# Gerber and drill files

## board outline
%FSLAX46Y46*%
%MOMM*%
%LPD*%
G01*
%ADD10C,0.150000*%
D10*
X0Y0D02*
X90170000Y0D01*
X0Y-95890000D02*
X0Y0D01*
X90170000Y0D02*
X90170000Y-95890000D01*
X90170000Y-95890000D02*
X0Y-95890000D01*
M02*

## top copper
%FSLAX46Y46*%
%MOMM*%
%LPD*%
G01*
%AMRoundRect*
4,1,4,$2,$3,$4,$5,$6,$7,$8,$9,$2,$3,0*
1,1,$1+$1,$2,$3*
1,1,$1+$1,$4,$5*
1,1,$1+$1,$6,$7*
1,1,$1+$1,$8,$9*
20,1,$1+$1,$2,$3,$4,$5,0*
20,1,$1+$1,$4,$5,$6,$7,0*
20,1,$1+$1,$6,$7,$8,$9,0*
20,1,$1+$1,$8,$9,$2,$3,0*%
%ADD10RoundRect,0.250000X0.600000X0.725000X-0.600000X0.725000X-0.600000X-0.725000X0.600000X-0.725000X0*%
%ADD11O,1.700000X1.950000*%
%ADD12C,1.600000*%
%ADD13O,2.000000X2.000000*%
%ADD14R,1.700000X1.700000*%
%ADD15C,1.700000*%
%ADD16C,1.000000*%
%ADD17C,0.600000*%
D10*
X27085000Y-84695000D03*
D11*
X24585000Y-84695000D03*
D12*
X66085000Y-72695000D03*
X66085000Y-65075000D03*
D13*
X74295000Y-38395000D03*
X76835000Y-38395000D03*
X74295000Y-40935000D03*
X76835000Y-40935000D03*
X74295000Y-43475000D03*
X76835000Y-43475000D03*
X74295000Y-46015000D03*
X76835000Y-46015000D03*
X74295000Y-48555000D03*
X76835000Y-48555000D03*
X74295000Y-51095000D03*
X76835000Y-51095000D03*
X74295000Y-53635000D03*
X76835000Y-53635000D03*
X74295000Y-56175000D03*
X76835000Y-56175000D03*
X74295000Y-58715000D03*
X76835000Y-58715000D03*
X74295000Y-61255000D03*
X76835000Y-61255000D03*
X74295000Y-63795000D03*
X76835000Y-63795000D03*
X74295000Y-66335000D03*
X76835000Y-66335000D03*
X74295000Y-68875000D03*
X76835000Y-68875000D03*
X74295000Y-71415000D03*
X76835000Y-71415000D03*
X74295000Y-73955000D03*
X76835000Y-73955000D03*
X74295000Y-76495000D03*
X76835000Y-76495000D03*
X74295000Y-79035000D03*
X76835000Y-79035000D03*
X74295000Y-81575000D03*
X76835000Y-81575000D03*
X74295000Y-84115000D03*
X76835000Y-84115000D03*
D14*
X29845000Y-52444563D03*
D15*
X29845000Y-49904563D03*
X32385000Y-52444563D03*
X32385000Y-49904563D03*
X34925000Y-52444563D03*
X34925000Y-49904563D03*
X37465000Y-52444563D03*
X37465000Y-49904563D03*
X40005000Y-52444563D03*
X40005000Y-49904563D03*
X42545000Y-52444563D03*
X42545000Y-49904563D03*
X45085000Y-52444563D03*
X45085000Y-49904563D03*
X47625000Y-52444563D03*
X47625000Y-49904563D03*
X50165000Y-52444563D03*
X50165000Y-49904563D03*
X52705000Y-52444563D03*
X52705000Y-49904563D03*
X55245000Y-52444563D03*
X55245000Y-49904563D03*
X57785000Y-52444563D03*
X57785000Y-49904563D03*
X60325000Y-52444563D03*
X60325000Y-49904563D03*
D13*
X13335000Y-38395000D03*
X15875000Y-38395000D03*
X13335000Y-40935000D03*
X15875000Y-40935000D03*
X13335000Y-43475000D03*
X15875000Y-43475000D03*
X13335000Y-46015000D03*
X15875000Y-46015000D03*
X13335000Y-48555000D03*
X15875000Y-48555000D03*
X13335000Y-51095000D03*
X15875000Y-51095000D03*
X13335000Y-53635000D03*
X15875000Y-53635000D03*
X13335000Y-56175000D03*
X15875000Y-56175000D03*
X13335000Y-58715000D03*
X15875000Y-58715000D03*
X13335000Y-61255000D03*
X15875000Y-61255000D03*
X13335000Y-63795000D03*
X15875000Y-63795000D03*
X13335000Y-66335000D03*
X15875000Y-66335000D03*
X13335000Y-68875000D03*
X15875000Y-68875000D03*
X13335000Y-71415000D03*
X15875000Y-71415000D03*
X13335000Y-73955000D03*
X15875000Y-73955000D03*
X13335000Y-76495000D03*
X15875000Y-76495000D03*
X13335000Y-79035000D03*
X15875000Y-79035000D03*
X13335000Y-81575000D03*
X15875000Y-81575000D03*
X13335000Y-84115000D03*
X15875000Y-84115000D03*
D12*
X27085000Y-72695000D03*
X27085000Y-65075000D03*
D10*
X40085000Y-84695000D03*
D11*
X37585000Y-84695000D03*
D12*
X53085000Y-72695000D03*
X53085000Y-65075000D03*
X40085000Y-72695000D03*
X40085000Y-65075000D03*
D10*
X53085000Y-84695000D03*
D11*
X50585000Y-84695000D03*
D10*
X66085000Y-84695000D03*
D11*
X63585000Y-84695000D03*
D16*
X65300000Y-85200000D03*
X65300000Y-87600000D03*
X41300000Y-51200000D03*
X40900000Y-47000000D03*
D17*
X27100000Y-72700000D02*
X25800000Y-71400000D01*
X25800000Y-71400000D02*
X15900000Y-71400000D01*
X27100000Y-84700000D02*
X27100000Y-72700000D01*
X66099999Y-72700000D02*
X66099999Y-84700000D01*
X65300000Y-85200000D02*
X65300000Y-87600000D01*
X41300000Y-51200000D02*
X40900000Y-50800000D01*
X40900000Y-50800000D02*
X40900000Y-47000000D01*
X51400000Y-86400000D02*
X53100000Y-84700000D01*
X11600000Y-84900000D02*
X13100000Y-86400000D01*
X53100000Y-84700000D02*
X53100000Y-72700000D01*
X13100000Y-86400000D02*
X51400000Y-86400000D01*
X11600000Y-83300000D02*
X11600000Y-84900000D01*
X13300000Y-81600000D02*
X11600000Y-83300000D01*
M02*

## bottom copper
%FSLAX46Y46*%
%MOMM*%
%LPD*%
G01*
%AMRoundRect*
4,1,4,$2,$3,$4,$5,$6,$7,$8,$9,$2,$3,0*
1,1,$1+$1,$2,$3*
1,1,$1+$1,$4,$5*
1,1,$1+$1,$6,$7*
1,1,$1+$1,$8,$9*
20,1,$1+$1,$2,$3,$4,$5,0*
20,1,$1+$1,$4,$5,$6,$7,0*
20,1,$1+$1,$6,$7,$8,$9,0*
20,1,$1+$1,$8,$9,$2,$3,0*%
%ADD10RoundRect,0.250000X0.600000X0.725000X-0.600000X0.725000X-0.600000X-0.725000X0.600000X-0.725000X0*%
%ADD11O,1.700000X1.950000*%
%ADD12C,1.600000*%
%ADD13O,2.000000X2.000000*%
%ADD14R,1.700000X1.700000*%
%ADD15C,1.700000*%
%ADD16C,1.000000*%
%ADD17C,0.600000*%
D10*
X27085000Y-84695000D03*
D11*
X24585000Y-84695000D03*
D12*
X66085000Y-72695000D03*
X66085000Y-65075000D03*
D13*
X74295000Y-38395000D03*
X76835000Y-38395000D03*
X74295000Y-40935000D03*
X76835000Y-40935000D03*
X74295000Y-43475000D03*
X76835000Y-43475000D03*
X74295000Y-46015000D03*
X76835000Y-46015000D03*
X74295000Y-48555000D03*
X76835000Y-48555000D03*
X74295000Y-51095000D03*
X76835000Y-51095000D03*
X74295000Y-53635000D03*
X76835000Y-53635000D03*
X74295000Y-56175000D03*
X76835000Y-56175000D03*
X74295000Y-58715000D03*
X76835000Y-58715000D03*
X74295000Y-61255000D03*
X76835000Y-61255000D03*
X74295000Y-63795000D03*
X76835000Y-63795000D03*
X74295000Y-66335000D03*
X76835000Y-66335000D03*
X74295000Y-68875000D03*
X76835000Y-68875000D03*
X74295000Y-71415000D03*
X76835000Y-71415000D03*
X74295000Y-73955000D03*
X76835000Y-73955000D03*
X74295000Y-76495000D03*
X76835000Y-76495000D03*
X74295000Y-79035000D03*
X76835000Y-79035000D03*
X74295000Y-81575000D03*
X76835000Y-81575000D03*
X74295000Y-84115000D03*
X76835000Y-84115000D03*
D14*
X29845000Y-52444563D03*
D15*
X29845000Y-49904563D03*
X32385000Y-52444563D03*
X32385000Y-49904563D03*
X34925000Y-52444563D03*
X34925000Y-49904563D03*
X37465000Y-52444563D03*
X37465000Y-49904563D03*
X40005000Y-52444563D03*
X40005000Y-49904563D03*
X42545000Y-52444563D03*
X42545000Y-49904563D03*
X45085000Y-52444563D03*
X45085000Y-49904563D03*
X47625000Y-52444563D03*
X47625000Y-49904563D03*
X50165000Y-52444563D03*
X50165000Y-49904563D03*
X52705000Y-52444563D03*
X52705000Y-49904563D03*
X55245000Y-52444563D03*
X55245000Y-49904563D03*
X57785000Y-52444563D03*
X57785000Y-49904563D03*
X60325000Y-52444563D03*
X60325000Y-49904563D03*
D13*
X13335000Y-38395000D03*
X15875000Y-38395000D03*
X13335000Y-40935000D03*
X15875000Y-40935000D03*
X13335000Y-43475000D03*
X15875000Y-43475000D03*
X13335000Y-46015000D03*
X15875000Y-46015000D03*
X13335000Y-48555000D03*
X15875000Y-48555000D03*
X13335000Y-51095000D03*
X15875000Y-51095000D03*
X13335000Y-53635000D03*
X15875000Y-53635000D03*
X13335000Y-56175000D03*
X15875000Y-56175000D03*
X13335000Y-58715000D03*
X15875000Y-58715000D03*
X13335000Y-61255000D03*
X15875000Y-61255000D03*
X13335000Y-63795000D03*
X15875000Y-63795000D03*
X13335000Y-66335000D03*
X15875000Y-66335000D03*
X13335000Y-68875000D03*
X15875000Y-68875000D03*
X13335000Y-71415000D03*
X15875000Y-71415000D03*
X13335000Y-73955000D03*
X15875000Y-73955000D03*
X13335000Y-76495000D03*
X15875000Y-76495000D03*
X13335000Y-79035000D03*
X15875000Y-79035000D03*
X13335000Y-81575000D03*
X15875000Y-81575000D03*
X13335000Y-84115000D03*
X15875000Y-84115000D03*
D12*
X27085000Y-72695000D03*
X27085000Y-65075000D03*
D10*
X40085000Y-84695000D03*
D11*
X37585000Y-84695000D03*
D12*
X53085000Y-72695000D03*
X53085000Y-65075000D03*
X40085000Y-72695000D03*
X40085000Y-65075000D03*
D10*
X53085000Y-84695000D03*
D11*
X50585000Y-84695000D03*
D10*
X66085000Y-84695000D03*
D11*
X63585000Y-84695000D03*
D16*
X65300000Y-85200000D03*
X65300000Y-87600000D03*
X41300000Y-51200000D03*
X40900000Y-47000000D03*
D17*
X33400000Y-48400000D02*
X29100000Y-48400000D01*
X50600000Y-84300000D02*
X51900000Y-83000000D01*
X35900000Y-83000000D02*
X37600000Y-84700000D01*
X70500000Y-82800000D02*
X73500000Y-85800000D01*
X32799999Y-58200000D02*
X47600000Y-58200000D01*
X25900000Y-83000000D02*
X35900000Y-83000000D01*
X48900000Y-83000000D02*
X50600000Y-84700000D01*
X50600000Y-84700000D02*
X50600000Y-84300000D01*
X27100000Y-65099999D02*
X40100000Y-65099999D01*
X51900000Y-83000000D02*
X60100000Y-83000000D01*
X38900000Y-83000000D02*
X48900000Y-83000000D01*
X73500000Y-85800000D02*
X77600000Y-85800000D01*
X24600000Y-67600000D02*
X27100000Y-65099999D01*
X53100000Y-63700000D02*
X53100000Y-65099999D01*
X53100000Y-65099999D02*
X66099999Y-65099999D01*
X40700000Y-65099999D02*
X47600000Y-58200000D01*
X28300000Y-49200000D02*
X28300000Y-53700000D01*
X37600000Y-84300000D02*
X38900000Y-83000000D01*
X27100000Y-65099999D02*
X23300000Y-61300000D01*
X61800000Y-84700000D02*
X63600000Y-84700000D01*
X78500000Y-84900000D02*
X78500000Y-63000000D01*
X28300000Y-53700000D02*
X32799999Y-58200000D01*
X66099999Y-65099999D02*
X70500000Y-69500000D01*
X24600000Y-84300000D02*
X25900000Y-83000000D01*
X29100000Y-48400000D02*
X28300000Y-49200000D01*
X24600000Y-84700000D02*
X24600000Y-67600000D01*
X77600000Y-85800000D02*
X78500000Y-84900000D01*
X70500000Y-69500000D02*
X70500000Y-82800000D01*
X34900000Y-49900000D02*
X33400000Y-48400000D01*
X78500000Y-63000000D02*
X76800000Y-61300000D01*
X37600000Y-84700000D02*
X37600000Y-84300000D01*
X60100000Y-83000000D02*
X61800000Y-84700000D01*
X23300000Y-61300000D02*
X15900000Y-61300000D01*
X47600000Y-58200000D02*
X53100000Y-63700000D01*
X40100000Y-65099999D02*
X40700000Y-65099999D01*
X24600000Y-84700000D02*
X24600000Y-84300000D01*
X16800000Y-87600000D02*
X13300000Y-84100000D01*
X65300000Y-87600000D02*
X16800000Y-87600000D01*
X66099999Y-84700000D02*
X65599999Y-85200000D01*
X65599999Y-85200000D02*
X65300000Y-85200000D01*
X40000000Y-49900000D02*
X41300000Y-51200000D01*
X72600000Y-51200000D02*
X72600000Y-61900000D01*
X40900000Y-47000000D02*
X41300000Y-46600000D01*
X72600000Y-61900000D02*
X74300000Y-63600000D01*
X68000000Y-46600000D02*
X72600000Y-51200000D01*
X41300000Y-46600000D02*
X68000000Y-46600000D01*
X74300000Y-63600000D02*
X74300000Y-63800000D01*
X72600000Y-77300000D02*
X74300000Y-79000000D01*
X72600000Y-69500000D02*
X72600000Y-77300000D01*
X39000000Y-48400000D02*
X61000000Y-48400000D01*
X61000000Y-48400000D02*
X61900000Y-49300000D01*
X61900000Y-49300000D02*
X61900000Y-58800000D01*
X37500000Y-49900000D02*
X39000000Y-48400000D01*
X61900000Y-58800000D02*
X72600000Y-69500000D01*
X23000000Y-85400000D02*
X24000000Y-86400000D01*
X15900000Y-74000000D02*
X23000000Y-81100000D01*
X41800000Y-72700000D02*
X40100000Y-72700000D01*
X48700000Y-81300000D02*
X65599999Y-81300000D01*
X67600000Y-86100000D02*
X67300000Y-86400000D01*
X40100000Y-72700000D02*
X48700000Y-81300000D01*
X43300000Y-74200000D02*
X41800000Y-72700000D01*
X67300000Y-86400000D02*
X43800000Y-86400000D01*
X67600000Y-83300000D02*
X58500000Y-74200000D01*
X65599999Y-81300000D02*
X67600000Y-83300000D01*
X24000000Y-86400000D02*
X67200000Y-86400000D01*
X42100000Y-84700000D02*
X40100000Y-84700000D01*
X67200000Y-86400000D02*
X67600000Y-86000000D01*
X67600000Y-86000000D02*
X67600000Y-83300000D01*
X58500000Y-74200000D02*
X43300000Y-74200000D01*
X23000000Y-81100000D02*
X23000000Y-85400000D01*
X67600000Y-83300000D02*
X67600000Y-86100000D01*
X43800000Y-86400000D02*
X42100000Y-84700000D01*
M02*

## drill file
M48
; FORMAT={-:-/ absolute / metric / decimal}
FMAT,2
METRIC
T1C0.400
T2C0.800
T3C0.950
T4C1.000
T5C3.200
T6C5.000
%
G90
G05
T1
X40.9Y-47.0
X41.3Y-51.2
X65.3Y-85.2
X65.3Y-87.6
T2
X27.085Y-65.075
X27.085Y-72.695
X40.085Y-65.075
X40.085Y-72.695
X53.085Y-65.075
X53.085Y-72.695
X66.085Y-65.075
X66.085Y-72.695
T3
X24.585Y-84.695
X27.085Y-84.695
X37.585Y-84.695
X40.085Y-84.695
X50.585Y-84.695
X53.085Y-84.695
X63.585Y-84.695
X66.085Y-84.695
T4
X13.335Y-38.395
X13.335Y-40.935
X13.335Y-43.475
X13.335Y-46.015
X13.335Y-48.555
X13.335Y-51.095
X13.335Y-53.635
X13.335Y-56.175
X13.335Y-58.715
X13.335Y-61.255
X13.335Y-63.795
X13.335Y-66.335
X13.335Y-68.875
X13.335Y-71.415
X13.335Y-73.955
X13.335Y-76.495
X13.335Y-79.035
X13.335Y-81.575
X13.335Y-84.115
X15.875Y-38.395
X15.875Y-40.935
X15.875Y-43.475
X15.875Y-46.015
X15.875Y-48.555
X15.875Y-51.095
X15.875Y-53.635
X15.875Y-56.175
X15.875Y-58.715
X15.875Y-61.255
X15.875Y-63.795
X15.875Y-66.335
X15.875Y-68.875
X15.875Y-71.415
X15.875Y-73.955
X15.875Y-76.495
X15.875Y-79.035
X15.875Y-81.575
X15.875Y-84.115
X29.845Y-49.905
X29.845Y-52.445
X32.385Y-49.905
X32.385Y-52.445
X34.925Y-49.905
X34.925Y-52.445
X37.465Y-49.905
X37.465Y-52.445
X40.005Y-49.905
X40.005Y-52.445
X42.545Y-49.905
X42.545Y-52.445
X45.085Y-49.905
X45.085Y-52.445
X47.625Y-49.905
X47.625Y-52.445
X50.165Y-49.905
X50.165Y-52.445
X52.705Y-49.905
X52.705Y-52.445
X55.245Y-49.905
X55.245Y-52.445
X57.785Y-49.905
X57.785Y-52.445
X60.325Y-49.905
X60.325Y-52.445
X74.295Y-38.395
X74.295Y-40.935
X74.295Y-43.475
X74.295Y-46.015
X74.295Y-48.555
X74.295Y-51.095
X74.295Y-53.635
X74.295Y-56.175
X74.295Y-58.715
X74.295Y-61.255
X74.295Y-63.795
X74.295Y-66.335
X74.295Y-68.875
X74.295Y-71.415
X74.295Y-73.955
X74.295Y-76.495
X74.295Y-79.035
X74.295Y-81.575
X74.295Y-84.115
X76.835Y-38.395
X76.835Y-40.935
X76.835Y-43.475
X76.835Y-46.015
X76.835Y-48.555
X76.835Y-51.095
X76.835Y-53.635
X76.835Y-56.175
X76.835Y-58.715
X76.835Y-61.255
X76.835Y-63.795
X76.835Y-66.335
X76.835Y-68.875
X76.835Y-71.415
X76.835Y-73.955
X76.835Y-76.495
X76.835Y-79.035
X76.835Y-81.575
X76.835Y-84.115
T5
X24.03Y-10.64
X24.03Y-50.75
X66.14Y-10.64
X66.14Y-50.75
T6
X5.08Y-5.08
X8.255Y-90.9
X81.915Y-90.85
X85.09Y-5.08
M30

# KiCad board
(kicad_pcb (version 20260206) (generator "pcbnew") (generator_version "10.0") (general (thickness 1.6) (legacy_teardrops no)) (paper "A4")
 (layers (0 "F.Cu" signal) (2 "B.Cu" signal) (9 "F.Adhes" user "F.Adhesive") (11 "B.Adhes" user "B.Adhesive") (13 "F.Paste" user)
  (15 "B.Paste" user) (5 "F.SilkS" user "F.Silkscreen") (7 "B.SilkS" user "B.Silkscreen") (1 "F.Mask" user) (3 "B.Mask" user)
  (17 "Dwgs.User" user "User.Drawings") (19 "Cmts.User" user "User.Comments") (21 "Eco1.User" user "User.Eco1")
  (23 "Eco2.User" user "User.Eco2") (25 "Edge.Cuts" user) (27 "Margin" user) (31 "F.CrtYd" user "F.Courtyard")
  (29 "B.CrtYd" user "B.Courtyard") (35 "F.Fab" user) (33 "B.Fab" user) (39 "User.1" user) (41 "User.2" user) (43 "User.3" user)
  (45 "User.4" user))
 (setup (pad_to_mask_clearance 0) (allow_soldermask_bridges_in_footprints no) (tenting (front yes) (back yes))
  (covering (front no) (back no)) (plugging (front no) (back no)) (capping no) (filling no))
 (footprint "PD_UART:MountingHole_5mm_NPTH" (layer "F.Cu") (at 8.255 90.9)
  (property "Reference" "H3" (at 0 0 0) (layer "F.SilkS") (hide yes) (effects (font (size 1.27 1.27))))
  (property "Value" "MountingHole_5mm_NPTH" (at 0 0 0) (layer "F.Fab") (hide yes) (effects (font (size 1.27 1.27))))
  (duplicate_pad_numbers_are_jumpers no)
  (pad "" np_thru_hole circle (at 0 0) (size 5 5) (drill 5) (layers "*.Cu")))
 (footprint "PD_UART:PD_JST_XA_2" (layer "F.Cu") (at 27.085 84.695 180)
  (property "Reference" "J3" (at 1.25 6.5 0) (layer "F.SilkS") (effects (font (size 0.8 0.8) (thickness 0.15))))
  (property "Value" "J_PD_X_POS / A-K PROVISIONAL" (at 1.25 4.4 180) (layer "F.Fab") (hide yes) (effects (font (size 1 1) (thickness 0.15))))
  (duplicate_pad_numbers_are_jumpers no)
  (pad "1" thru_hole roundrect (at 0 0 180) (size 1.7 1.95) (drill 0.95) (layers "*.Cu") (remove_unused_layers no)
   (roundrect_rratio 0.147059) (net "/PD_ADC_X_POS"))
  (pad "2" thru_hole oval (at 2.5 0 180) (size 1.7 1.95) (drill 0.95) (layers "*.Cu") (remove_unused_layers no) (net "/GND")))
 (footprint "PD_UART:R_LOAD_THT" (layer "F.Cu") (at 66.085 72.695 90)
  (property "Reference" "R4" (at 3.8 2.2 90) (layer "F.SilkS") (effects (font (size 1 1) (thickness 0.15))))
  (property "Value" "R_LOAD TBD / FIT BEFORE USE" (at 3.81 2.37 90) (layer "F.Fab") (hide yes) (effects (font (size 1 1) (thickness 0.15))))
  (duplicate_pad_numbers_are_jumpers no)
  (pad "1" thru_hole circle (at 0 0 90) (size 1.6 1.6) (drill 0.8) (layers "*.Cu") (remove_unused_layers no) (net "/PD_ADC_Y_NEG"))
  (pad "2" thru_hole circle (at 7.62 0 90) (size 1.6 1.6) (drill 0.8) (layers "*.Cu") (remove_unused_layers no) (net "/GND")))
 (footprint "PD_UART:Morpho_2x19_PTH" (layer "F.Cu") (at 74.295 38.395)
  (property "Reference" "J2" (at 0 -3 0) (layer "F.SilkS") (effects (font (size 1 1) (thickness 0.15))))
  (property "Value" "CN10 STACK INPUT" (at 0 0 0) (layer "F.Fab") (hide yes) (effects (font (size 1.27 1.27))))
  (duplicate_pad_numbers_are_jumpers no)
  (pad "1" thru_hole oval (at 0 0) (size 2 2) (drill 1) (layers "*.Cu") (remove_unused_layers no) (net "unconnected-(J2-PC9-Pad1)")
   (thermal_bridge_angle 45))
  (pad "2" thru_hole oval (at 2.54 0) (size 2 2) (drill 1) (layers "*.Cu") (remove_unused_layers no) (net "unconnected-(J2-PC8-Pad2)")
   (thermal_bridge_angle 45))
  (pad "3" thru_hole oval (at 0 2.54) (size 2 2) (drill 1) (layers "*.Cu") (remove_unused_layers no) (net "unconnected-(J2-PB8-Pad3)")
   (thermal_bridge_angle 45))
  (pad "4" thru_hole oval (at 2.54 2.54) (size 2 2) (drill 1) (layers "*.Cu") (remove_unused_layers no) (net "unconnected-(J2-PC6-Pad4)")
   (thermal_bridge_angle 45))
  (pad "5" thru_hole oval (at 0 5.08) (size 2 2) (drill 1) (layers "*.Cu") (remove_unused_layers no) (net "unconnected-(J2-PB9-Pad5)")
   (thermal_bridge_angle 45))
  (pad "6" thru_hole oval (at 2.54 5.08) (size 2 2) (drill 1) (layers "*.Cu") (remove_unused_layers no) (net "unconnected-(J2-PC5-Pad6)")
   (thermal_bridge_angle 45))
  (pad "7" thru_hole oval (at 0 7.62) (size 2 2) (drill 1) (layers "*.Cu") (remove_unused_layers no) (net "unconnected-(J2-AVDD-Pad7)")
   (thermal_bridge_angle 45))
  (pad "8" thru_hole oval (at 2.54 7.62) (size 2 2) (drill 1) (layers "*.Cu") (remove_unused_layers no) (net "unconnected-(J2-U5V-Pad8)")
   (thermal_bridge_angle 45))
  (pad "9" thru_hole oval (at 0 10.16) (size 2 2) (drill 1) (layers "*.Cu") (remove_unused_layers no) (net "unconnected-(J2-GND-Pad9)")
   (thermal_bridge_angle 45))
  (pad "10" thru_hole oval (at 2.54 10.16) (size 2 2) (drill 1) (layers "*.Cu") (remove_unused_layers no) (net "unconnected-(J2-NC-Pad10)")
   (thermal_bridge_angle 45))
  (pad "11" thru_hole oval (at 0 12.7) (size 2 2) (drill 1) (layers "*.Cu") (remove_unused_layers no) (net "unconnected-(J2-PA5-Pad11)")
   (thermal_bridge_angle 45))
  (pad "12" thru_hole oval (at 2.54 12.7) (size 2 2) (drill 1) (layers "*.Cu") (remove_unused_layers no) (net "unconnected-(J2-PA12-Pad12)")
   (thermal_bridge_angle 45))
  (pad "13" thru_hole oval (at 0 15.24) (size 2 2) (drill 1) (layers "*.Cu") (remove_unused_layers no) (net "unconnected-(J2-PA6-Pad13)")
   (thermal_bridge_angle 45))
  (pad "14" thru_hole oval (at 2.54 15.24) (size 2 2) (drill 1) (layers "*.Cu") (remove_unused_layers no)
   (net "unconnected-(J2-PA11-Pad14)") (thermal_bridge_angle 45))
  (pad "15" thru_hole oval (at 0 17.78) (size 2 2) (drill 1) (layers "*.Cu") (remove_unused_layers no) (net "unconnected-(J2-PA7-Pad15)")
   (thermal_bridge_angle 45))
  (pad "16" thru_hole oval (at 2.54 17.78) (size 2 2) (drill 1) (layers "*.Cu") (remove_unused_layers no)
   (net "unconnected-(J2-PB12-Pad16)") (thermal_bridge_angle 45))
  (pad "17" thru_hole oval (at 0 20.32) (size 2 2) (drill 1) (layers "*.Cu") (remove_unused_layers no) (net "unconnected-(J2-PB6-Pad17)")
   (thermal_bridge_angle 45))
  (pad "18" thru_hole oval (at 2.54 20.32) (size 2 2) (drill 1) (layers "*.Cu") (remove_unused_layers no)
   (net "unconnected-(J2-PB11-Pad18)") (thermal_bridge_angle 45))
  (pad "19" thru_hole oval (at 0 22.86) (size 2 2) (drill 1) (layers "*.Cu") (remove_unused_layers no) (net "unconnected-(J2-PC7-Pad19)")
   (thermal_bridge_angle 45))
  (pad "20" thru_hole oval (at 2.54 22.86) (size 2 2) (drill 1) (layers "*.Cu") (remove_unused_layers no) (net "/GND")
   (thermal_bridge_angle 45))
  (pad "21" thru_hole oval (at 0 25.4) (size 2 2) (drill 1) (layers "*.Cu") (remove_unused_layers no) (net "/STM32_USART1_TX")
   (thermal_bridge_angle 45))
  (pad "22" thru_hole oval (at 2.54 25.4) (size 2 2) (drill 1) (layers "*.Cu") (remove_unused_layers no) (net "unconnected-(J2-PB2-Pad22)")
   (thermal_bridge_angle 45))
  (pad "23" thru_hole oval (at 0 27.94) (size 2 2) (drill 1) (layers "*.Cu") (remove_unused_layers no) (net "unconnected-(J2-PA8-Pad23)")
   (thermal_bridge_angle 45))
  (pad "24" thru_hole oval (at 2.54 27.94) (size 2 2) (drill 1) (layers "*.Cu") (remove_unused_layers no) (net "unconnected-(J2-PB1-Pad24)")
   (thermal_bridge_angle 45))
  (pad "25" thru_hole oval (at 0 30.48) (size 2 2) (drill 1) (layers "*.Cu") (remove_unused_layers no) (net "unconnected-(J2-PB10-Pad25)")
   (thermal_bridge_angle 45))
  (pad "26" thru_hole oval (at 2.54 30.48) (size 2 2) (drill 1) (layers "*.Cu") (remove_unused_layers no)
   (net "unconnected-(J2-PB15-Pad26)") (thermal_bridge_angle 45))
  (pad "27" thru_hole oval (at 0 33.02) (size 2 2) (drill 1) (layers "*.Cu") (remove_unused_layers no) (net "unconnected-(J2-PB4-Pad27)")
   (thermal_bridge_angle 45))
  (pad "28" thru_hole oval (at 2.54 33.02) (size 2 2) (drill 1) (layers "*.Cu") (remove_unused_layers no)
   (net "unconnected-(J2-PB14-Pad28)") (thermal_bridge_angle 45))
  (pad "29" thru_hole oval (at 0 35.56) (size 2 2) (drill 1) (layers "*.Cu") (remove_unused_layers no) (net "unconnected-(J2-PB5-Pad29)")
   (thermal_bridge_angle 45))
  (pad "30" thru_hole oval (at 2.54 35.56) (size 2 2) (drill 1) (layers "*.Cu") (remove_unused_layers no)
   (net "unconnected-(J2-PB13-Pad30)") (thermal_bridge_angle 45))
  (pad "31" thru_hole oval (at 0 38.1) (size 2 2) (drill 1) (layers "*.Cu") (remove_unused_layers no) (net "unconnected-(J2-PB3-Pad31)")
   (thermal_bridge_angle 45))
  (pad "32" thru_hole oval (at 2.54 38.1) (size 2 2) (drill 1) (layers "*.Cu") (remove_unused_layers no) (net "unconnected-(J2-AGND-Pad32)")
   (thermal_bridge_angle 45))
  (pad "33" thru_hole oval (at 0 40.64) (size 2 2) (drill 1) (layers "*.Cu") (remove_unused_layers no) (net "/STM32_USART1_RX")
   (thermal_bridge_angle 45))
  (pad "34" thru_hole oval (at 2.54 40.64) (size 2 2) (drill 1) (layers "*.Cu") (remove_unused_layers no) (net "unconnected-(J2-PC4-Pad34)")
   (thermal_bridge_angle 45))
  (pad "35" thru_hole oval (at 0 43.18) (size 2 2) (drill 1) (layers "*.Cu") (remove_unused_layers no) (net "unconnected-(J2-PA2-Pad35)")
   (thermal_bridge_angle 45))
  (pad "36" thru_hole oval (at 2.54 43.18) (size 2 2) (drill 1) (layers "*.Cu") (remove_unused_layers no) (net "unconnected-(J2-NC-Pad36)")
   (thermal_bridge_angle 45))
  (pad "37" thru_hole oval (at 0 45.72) (size 2 2) (drill 1) (layers "*.Cu") (remove_unused_layers no) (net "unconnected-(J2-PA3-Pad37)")
   (thermal_bridge_angle 45))
  (pad "38" thru_hole oval (at 2.54 45.72) (size 2 2) (drill 1) (layers "*.Cu") (remove_unused_layers no) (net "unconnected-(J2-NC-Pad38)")
   (thermal_bridge_angle 45)))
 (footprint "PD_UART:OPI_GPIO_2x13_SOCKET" (layer "F.Cu") (at 29.845 52.444563)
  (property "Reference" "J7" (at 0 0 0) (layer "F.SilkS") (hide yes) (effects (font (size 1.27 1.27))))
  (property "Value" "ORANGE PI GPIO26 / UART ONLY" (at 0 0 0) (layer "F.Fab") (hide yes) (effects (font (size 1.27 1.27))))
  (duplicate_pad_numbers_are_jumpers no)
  (pad "1" thru_hole rect (at 0 0) (size 1.7 1.7) (drill 1) (layers "*.Cu") (remove_unused_layers no) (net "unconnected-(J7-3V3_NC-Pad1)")
   (thermal_bridge_angle 45))
  (pad "2" thru_hole circle (at 0 -2.54) (size 1.7 1.7) (drill 1) (layers "*.Cu") (remove_unused_layers no)
   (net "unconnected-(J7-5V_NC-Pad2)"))
  (pad "3" thru_hole circle (at 2.54 0) (size 1.7 1.7) (drill 1) (layers "*.Cu") (remove_unused_layers no)
   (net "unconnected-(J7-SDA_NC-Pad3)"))
  (pad "4" thru_hole circle (at 2.54 -2.54) (size 1.7 1.7) (drill 1) (layers "*.Cu") (remove_unused_layers no)
   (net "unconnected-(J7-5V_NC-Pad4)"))
  (pad "5" thru_hole circle (at 5.08 0) (size 1.7 1.7) (drill 1) (layers "*.Cu") (remove_unused_layers no)
   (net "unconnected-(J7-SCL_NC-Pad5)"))
  (pad "6" thru_hole circle (at 5.08 -2.54) (size 1.7 1.7) (drill 1) (layers "*.Cu") (remove_unused_layers no) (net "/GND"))
  (pad "7" thru_hole circle (at 7.62 0) (size 1.7 1.7) (drill 1) (layers "*.Cu") (remove_unused_layers no)
   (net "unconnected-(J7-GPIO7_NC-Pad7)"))
  (pad "8" thru_hole circle (at 7.62 -2.54) (size 1.7 1.7) (drill 1) (layers "*.Cu") (remove_unused_layers no) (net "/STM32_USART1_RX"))
  (pad "9" thru_hole circle (at 10.16 0) (size 1.7 1.7) (drill 1) (layers "*.Cu") (remove_unused_layers no)
   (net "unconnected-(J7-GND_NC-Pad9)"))
  (pad "10" thru_hole circle (at 10.16 -2.54) (size 1.7 1.7) (drill 1) (layers "*.Cu") (remove_unused_layers no) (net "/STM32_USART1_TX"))
  (pad "11" thru_hole circle (at 12.7 0) (size 1.7 1.7) (drill 1) (layers "*.Cu") (remove_unused_layers no)
   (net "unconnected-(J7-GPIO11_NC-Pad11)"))
  (pad "12" thru_hole circle (at 12.7 -2.54) (size 1.7 1.7) (drill 1) (layers "*.Cu") (remove_unused_layers no)
   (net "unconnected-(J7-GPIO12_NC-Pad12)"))
  (pad "13" thru_hole circle (at 15.24 0) (size 1.7 1.7) (drill 1) (layers "*.Cu") (remove_unused_layers no)
   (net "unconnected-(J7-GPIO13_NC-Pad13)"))
  (pad "14" thru_hole circle (at 15.24 -2.54) (size 1.7 1.7) (drill 1) (layers "*.Cu") (remove_unused_layers no)
   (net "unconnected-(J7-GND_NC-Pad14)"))
  (pad "15" thru_hole circle (at 17.78 0) (size 1.7 1.7) (drill 1) (layers "*.Cu") (remove_unused_layers no)
   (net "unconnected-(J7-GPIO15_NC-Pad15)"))
  (pad "16" thru_hole circle (at 17.78 -2.54) (size 1.7 1.7) (drill 1) (layers "*.Cu") (remove_unused_layers no)
   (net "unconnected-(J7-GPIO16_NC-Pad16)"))
  (pad "17" thru_hole circle (at 20.32 0) (size 1.7 1.7) (drill 1) (layers "*.Cu") (remove_unused_layers no)
   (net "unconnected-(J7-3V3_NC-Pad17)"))
  (pad "18" thru_hole circle (at 20.32 -2.54) (size 1.7 1.7) (drill 1) (layers "*.Cu") (remove_unused_layers no)
   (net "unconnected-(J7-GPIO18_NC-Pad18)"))
  (pad "19" thru_hole circle (at 22.86 0) (size 1.7 1.7) (drill 1) (layers "*.Cu") (remove_unused_layers no)
   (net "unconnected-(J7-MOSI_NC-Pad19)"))
  (pad "20" thru_hole circle (at 22.86 -2.54) (size 1.7 1.7) (drill 1) (layers "*.Cu") (remove_unused_layers no)
   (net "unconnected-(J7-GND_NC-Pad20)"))
  (pad "21" thru_hole circle (at 25.4 0) (size 1.7 1.7) (drill 1) (layers "*.Cu") (remove_unused_layers no)
   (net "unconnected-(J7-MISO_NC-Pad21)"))
  (pad "22" thru_hole circle (at 25.4 -2.54) (size 1.7 1.7) (drill 1) (layers "*.Cu") (remove_unused_layers no)
   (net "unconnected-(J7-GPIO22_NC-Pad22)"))
  (pad "23" thru_hole circle (at 27.94 0) (size 1.7 1.7) (drill 1) (layers "*.Cu") (remove_unused_layers no)
   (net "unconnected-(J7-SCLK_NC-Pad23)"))
  (pad "24" thru_hole circle (at 27.94 -2.54) (size 1.7 1.7) (drill 1) (layers "*.Cu") (remove_unused_layers no)
   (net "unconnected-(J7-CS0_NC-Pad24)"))
  (pad "25" thru_hole circle (at 30.48 0) (size 1.7 1.7) (drill 1) (layers "*.Cu") (remove_unused_layers no)
   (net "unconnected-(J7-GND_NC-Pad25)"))
  (pad "26" thru_hole circle (at 30.48 -2.54) (size 1.7 1.7) (drill 1) (layers "*.Cu") (remove_unused_layers no)
   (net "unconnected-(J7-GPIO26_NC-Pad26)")))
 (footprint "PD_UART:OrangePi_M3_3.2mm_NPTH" (layer "F.Cu") (at 66.140457 10.639541)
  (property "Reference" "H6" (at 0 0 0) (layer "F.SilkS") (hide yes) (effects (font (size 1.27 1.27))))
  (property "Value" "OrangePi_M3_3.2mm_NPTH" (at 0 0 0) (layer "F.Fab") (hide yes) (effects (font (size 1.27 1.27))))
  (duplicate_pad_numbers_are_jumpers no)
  (pad "" np_thru_hole circle (at 0 0) (size 3.2 3.2) (drill 3.2) (layers "*.Cu")))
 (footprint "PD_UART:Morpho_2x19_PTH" (layer "F.Cu") (at 13.335 38.395)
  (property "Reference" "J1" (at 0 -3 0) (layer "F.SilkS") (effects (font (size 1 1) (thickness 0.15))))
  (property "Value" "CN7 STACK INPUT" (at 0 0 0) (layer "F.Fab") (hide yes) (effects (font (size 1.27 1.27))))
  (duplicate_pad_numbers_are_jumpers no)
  (pad "1" thru_hole oval (at 0 0) (size 2 2) (drill 1) (layers "*.Cu") (remove_unused_layers no) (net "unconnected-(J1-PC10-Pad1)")
   (thermal_bridge_angle 45))
  (pad "2" thru_hole oval (at 2.54 0) (size 2 2) (drill 1) (layers "*.Cu") (remove_unused_layers no) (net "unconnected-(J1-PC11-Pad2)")
   (thermal_bridge_angle 45))
  (pad "3" thru_hole oval (at 0 2.54) (size 2 2) (drill 1) (layers "*.Cu") (remove_unused_layers no) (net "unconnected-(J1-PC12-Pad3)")
   (thermal_bridge_angle 45))
  (pad "4" thru_hole oval (at 2.54 2.54) (size 2 2) (drill 1) (layers "*.Cu") (remove_unused_layers no) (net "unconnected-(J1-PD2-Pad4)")
   (thermal_bridge_angle 45))
  (pad "5" thru_hole oval (at 0 5.08) (size 2 2) (drill 1) (layers "*.Cu") (remove_unused_layers no) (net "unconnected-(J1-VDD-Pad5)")
   (thermal_bridge_angle 45))
  (pad "6" thru_hole oval (at 2.54 5.08) (size 2 2) (drill 1) (layers "*.Cu") (remove_unused_layers no) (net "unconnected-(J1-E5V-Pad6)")
   (thermal_bridge_angle 45))
  (pad "7" thru_hole oval (at 0 7.62) (size 2 2) (drill 1) (layers "*.Cu") (remove_unused_layers no) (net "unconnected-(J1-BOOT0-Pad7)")
   (thermal_bridge_angle 45))
  (pad "8" thru_hole oval (at 2.54 7.62) (size 2 2) (drill 1) (layers "*.Cu") (remove_unused_layers no) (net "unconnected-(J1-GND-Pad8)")
   (thermal_bridge_angle 45))
  (pad "9" thru_hole oval (at 0 10.16) (size 2 2) (drill 1) (layers "*.Cu") (remove_unused_layers no) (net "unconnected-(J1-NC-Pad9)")
   (thermal_bridge_angle 45))
  (pad "10" thru_hole oval (at 2.54 10.16) (size 2 2) (drill 1) (layers "*.Cu") (remove_unused_layers no) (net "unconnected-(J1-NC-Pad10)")
   (thermal_bridge_angle 45))
  (pad "11" thru_hole oval (at 0 12.7) (size 2 2) (drill 1) (layers "*.Cu") (remove_unused_layers no) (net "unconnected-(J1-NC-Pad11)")
   (thermal_bridge_angle 45))
  (pad "12" thru_hole oval (at 2.54 12.7) (size 2 2) (drill 1) (layers "*.Cu") (remove_unused_layers no)
   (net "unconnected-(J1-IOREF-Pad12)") (thermal_bridge_angle 45))
  (pad "13" thru_hole oval (at 0 15.24) (size 2 2) (drill 1) (layers "*.Cu") (remove_unused_layers no) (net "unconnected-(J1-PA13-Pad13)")
   (thermal_bridge_angle 45))
  (pad "14" thru_hole oval (at 2.54 15.24) (size 2 2) (drill 1) (layers "*.Cu") (remove_unused_layers no)
   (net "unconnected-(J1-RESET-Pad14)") (thermal_bridge_angle 45))
  (pad "15" thru_hole oval (at 0 17.78) (size 2 2) (drill 1) (layers "*.Cu") (remove_unused_layers no) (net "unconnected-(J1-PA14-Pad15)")
   (thermal_bridge_angle 45))
  (pad "16" thru_hole oval (at 2.54 17.78) (size 2 2) (drill 1) (layers "*.Cu") (remove_unused_layers no) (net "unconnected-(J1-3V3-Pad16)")
   (thermal_bridge_angle 45))
  (pad "17" thru_hole oval (at 0 20.32) (size 2 2) (drill 1) (layers "*.Cu") (remove_unused_layers no) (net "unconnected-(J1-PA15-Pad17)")
   (thermal_bridge_angle 45))
  (pad "18" thru_hole oval (at 2.54 20.32) (size 2 2) (drill 1) (layers "*.Cu") (remove_unused_layers no) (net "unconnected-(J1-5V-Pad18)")
   (thermal_bridge_angle 45))
  (pad "19" thru_hole oval (at 0 22.86) (size 2 2) (drill 1) (layers "*.Cu") (remove_unused_layers no) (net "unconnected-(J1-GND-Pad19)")
   (thermal_bridge_angle 45))
  (pad "20" thru_hole oval (at 2.54 22.86) (size 2 2) (drill 1) (layers "*.Cu") (remove_unused_layers no) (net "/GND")
   (thermal_bridge_angle 45))
  (pad "21" thru_hole oval (at 0 25.4) (size 2 2) (drill 1) (layers "*.Cu") (remove_unused_layers no) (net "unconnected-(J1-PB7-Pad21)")
   (thermal_bridge_angle 45))
  (pad "22" thru_hole oval (at 2.54 25.4) (size 2 2) (drill 1) (layers "*.Cu") (remove_unused_layers no) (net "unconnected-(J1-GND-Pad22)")
   (thermal_bridge_angle 45))
  (pad "23" thru_hole oval (at 0 27.94) (size 2 2) (drill 1) (layers "*.Cu") (remove_unused_layers no) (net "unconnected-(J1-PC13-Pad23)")
   (thermal_bridge_angle 45))
  (pad "24" thru_hole oval (at 2.54 27.94) (size 2 2) (drill 1) (layers "*.Cu") (remove_unused_layers no) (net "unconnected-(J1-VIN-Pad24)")
   (thermal_bridge_angle 45))
  (pad "25" thru_hole oval (at 0 30.48) (size 2 2) (drill 1) (layers "*.Cu") (remove_unused_layers no) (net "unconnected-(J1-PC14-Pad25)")
   (thermal_bridge_angle 45))
  (pad "26" thru_hole oval (at 2.54 30.48) (size 2 2) (drill 1) (layers "*.Cu") (remove_unused_layers no) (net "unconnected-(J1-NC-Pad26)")
   (thermal_bridge_angle 45))
  (pad "27" thru_hole oval (at 0 33.02) (size 2 2) (drill 1) (layers "*.Cu") (remove_unused_layers no) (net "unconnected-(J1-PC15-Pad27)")
   (thermal_bridge_angle 45))
  (pad "28" thru_hole oval (at 2.54 33.02) (size 2 2) (drill 1) (layers "*.Cu") (remove_unused_layers no) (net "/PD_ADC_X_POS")
   (thermal_bridge_angle 45))
  (pad "29" thru_hole oval (at 0 35.56) (size 2 2) (drill 1) (layers "*.Cu") (remove_unused_layers no) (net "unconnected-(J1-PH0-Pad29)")
   (thermal_bridge_angle 45))
  (pad "30" thru_hole oval (at 2.54 35.56) (size 2 2) (drill 1) (layers "*.Cu") (remove_unused_layers no) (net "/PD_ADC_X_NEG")
   (thermal_bridge_angle 45))
  (pad "31" thru_hole oval (at 0 38.1) (size 2 2) (drill 1) (layers "*.Cu") (remove_unused_layers no) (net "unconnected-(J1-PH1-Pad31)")
   (thermal_bridge_angle 45))
  (pad "32" thru_hole oval (at 2.54 38.1) (size 2 2) (drill 1) (layers "*.Cu") (remove_unused_layers no) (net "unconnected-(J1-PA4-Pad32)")
   (thermal_bridge_angle 45))
  (pad "33" thru_hole oval (at 0 40.64) (size 2 2) (drill 1) (layers "*.Cu") (remove_unused_layers no) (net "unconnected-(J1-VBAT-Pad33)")
   (thermal_bridge_angle 45))
  (pad "34" thru_hole oval (at 2.54 40.64) (size 2 2) (drill 1) (layers "*.Cu") (remove_unused_layers no) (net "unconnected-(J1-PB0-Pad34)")
   (thermal_bridge_angle 45))
  (pad "35" thru_hole oval (at 0 43.18) (size 2 2) (drill 1) (layers "*.Cu") (remove_unused_layers no) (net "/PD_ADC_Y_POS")
   (thermal_bridge_angle 45))
  (pad "36" thru_hole oval (at 2.54 43.18) (size 2 2) (drill 1) (layers "*.Cu") (remove_unused_layers no)
   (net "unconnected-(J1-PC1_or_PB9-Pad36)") (thermal_bridge_angle 45))
  (pad "37" thru_hole oval (at 0 45.72) (size 2 2) (drill 1) (layers "*.Cu") (remove_unused_layers no) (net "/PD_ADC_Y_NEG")
   (thermal_bridge_angle 45))
  (pad "38" thru_hole oval (at 2.54 45.72) (size 2 2) (drill 1) (layers "*.Cu") (remove_unused_layers no) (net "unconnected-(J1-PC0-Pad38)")
   (thermal_bridge_angle 45)))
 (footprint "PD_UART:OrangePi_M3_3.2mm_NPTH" (layer "F.Cu") (at 24.029543 50.750459)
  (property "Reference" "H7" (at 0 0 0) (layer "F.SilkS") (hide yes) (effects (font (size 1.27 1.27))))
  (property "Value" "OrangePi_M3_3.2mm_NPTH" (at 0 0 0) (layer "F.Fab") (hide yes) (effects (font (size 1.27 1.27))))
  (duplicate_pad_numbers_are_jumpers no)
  (pad "" np_thru_hole circle (at 0 0) (size 3.2 3.2) (drill 3.2) (layers "*.Cu")))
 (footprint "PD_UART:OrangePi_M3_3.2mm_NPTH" (layer "F.Cu") (at 24.029543 10.639541)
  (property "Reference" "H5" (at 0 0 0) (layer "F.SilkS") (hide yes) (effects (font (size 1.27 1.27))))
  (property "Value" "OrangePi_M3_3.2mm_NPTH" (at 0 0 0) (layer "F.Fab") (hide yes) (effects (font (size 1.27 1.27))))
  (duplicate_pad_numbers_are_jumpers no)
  (pad "" np_thru_hole circle (at 0 0) (size 3.2 3.2) (drill 3.2) (layers "*.Cu")))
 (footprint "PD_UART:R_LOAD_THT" (layer "F.Cu") (at 27.085 72.695 90)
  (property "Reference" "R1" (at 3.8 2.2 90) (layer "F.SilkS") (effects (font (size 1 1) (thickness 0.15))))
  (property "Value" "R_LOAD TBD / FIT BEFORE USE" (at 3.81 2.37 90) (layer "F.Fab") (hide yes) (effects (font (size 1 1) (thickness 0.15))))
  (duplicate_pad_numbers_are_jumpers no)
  (pad "1" thru_hole circle (at 0 0 90) (size 1.6 1.6) (drill 0.8) (layers "*.Cu") (remove_unused_layers no) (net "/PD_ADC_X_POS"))
  (pad "2" thru_hole circle (at 7.62 0 90) (size 1.6 1.6) (drill 0.8) (layers "*.Cu") (remove_unused_layers no) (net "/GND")))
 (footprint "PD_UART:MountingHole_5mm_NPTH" (layer "F.Cu") (at 81.915 90.85)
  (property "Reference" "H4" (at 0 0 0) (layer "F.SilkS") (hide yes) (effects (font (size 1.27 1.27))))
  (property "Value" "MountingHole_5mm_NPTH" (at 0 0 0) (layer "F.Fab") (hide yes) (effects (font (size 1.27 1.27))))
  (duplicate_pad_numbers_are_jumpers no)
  (pad "" np_thru_hole circle (at 0 0) (size 5 5) (drill 5) (layers "*.Cu")))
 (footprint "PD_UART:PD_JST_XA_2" (layer "F.Cu") (at 40.085 84.695 180)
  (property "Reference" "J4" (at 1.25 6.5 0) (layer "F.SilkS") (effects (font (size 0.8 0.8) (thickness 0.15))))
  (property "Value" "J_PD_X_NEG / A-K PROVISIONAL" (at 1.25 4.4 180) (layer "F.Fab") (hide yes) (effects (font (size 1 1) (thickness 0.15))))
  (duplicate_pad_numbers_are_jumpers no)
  (pad "1" thru_hole roundrect (at 0 0 180) (size 1.7 1.95) (drill 0.95) (layers "*.Cu") (remove_unused_layers no)
   (roundrect_rratio 0.147059) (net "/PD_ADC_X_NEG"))
  (pad "2" thru_hole oval (at 2.5 0 180) (size 1.7 1.95) (drill 0.95) (layers "*.Cu") (remove_unused_layers no) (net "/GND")))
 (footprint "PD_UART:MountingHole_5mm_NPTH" (layer "F.Cu") (at 85.09 5.08)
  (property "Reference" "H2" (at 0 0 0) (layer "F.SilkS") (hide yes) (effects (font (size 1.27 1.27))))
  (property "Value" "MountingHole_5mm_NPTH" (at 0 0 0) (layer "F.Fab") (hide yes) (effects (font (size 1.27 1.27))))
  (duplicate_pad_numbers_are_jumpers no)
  (pad "" np_thru_hole circle (at 0 0) (size 5 5) (drill 5) (layers "*.Cu")))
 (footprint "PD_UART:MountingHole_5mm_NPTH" (layer "F.Cu") (at 5.08 5.08)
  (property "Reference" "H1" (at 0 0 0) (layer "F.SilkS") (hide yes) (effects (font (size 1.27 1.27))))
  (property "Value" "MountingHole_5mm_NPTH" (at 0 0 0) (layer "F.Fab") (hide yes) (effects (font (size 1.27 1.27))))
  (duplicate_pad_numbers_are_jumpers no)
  (pad "" np_thru_hole circle (at 0 0) (size 5 5) (drill 5) (layers "*.Cu")))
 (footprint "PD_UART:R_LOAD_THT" (layer "F.Cu") (at 53.085 72.695 90)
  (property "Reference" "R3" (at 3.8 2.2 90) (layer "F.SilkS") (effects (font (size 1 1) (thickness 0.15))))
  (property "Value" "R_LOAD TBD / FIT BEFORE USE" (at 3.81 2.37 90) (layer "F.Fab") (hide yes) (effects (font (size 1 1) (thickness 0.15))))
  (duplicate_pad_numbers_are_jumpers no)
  (pad "1" thru_hole circle (at 0 0 90) (size 1.6 1.6) (drill 0.8) (layers "*.Cu") (remove_unused_layers no) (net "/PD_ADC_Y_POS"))
  (pad "2" thru_hole circle (at 7.62 0 90) (size 1.6 1.6) (drill 0.8) (layers "*.Cu") (remove_unused_layers no) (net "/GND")))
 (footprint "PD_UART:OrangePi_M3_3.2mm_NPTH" (layer "F.Cu") (at 66.140457 50.750459)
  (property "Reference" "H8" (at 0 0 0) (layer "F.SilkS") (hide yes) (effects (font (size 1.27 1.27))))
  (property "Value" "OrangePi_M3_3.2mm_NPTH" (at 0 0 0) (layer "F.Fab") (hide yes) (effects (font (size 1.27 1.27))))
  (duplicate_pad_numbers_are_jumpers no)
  (pad "" np_thru_hole circle (at 0 0) (size 3.2 3.2) (drill 3.2) (layers "*.Cu")))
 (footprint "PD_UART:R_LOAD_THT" (layer "F.Cu") (at 40.085 72.695 90)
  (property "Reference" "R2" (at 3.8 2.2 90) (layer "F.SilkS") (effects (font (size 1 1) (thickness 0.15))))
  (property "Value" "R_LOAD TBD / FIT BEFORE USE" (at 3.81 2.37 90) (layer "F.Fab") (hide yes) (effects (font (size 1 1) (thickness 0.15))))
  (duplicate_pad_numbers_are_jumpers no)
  (pad "1" thru_hole circle (at 0 0 90) (size 1.6 1.6) (drill 0.8) (layers "*.Cu") (remove_unused_layers no) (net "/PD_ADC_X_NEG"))
  (pad "2" thru_hole circle (at 7.62 0 90) (size 1.6 1.6) (drill 0.8) (layers "*.Cu") (remove_unused_layers no) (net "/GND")))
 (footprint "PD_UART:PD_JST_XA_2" (layer "F.Cu") (at 53.085 84.695 180)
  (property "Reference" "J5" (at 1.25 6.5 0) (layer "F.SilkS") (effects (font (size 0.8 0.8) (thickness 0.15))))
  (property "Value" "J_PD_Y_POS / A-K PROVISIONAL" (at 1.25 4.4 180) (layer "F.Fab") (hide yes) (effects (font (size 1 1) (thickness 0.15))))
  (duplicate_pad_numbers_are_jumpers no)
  (pad "1" thru_hole roundrect (at 0 0 180) (size 1.7 1.95) (drill 0.95) (layers "*.Cu") (remove_unused_layers no)
   (roundrect_rratio 0.147059) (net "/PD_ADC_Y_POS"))
  (pad "2" thru_hole oval (at 2.5 0 180) (size 1.7 1.95) (drill 0.95) (layers "*.Cu") (remove_unused_layers no) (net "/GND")))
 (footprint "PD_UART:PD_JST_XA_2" (layer "F.Cu") (at 66.085 84.695 180)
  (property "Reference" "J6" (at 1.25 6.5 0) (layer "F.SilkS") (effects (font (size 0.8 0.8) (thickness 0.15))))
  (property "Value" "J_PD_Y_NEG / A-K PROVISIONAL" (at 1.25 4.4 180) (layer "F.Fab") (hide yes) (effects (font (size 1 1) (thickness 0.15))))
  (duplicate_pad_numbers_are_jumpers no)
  (pad "1" thru_hole roundrect (at 0 0 180) (size 1.7 1.95) (drill 0.95) (layers "*.Cu") (remove_unused_layers no)
   (roundrect_rratio 0.147059) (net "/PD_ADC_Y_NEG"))
  (pad "2" thru_hole oval (at 2.5 0 180) (size 1.7 1.95) (drill 0.95) (layers "*.Cu") (remove_unused_layers no) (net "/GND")))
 (gr_line (start 0 0) (end 90.17 0) (stroke (width 0.15) (type default)) (layer "Edge.Cuts"))
 (gr_line (start 0 95.89) (end 0 0) (stroke (width 0.15) (type default)) (layer "Edge.Cuts"))
 (gr_line (start 90.17 0) (end 90.17 95.89) (stroke (width 0.15) (type default)) (layer "Edge.Cuts"))
 (gr_line (start 90.17 95.89) (end 0 95.89) (stroke (width 0.15) (type default)) (layer "Edge.Cuts"))
 (segment (start 27.1 72.7) (end 25.8 71.4) (width 0.6) (layer "F.Cu") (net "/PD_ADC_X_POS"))
 (segment (start 25.8 71.4) (end 15.9 71.4) (width 0.6) (layer "F.Cu") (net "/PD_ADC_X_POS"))
 (segment (start 27.1 84.7) (end 27.1 72.7) (width 0.6) (layer "F.Cu") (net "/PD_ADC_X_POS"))
 (segment (start 33.4 48.4) (end 29.1 48.4) (width 0.6) (layer "B.Cu") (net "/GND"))
 (segment (start 50.6 84.3) (end 51.9 83) (width 0.6) (layer "B.Cu") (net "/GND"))
 (segment (start 35.9 83) (end 37.6 84.7) (width 0.6) (layer "B.Cu") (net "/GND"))
 (segment (start 70.5 82.8) (end 73.5 85.8) (width 0.6) (layer "B.Cu") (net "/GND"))
 (segment (start 32.799999 58.2) (end 47.6 58.2) (width 0.6) (layer "B.Cu") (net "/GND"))
 (segment (start 25.9 83) (end 35.9 83) (width 0.6) (layer "B.Cu") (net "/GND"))
 (segment (start 48.9 83) (end 50.6 84.7) (width 0.6) (layer "B.Cu") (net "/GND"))
 (segment (start 50.6 84.7) (end 50.6 84.3) (width 0.6) (layer "B.Cu") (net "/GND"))
 (segment (start 27.1 65.099999) (end 40.1 65.099999) (width 0.6) (layer "B.Cu") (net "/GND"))
 (segment (start 51.9 83) (end 60.1 83) (width 0.6) (layer "B.Cu") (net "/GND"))
 (segment (start 38.9 83) (end 48.9 83) (width 0.6) (layer "B.Cu") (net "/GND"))
 (segment (start 73.5 85.8) (end 77.6 85.8) (width 0.6) (layer "B.Cu") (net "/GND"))
 (segment (start 24.6 67.6) (end 27.1 65.099999) (width 0.6) (layer "B.Cu") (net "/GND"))
 (segment (start 53.1 63.7) (end 53.1 65.099999) (width 0.6) (layer "B.Cu") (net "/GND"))
 (segment (start 53.1 65.099999) (end 66.099999 65.099999) (width 0.6) (layer "B.Cu") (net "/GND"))
 (segment (start 40.7 65.099999) (end 47.6 58.2) (width 0.6) (layer "B.Cu") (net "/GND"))
 (segment (start 28.3 49.2) (end 28.3 53.7) (width 0.6) (layer "B.Cu") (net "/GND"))
 (segment (start 37.6 84.3) (end 38.9 83) (width 0.6) (layer "B.Cu") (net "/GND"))
 (segment (start 27.1 65.099999) (end 23.3 61.3) (width 0.6) (layer "B.Cu") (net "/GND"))
 (segment (start 61.8 84.7) (end 63.6 84.7) (width 0.6) (layer "B.Cu") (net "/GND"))
 (segment (start 78.5 84.9) (end 78.5 63) (width 0.6) (layer "B.Cu") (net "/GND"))
 (segment (start 28.3 53.7) (end 32.799999 58.2) (width 0.6) (layer "B.Cu") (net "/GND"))
 (segment (start 66.099999 65.099999) (end 70.5 69.5) (width 0.6) (layer "B.Cu") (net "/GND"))
 (segment (start 24.6 84.3) (end 25.9 83) (width 0.6) (layer "B.Cu") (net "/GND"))
 (segment (start 29.1 48.4) (end 28.3 49.2) (width 0.6) (layer "B.Cu") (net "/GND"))
 (segment (start 24.6 84.7) (end 24.6 67.6) (width 0.6) (layer "B.Cu") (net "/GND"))
 (segment (start 77.6 85.8) (end 78.5 84.9) (width 0.6) (layer "B.Cu") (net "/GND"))
 (segment (start 70.5 69.5) (end 70.5 82.8) (width 0.6) (layer "B.Cu") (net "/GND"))
 (segment (start 34.9 49.9) (end 33.4 48.4) (width 0.6) (layer "B.Cu") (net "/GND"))
 (segment (start 78.5 63) (end 76.8 61.3) (width 0.6) (layer "B.Cu") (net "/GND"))
 (segment (start 37.6 84.7) (end 37.6 84.3) (width 0.6) (layer "B.Cu") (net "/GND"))
 (segment (start 60.1 83) (end 61.8 84.7) (width 0.6) (layer "B.Cu") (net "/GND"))
 (segment (start 23.3 61.3) (end 15.9 61.3) (width 0.6) (layer "B.Cu") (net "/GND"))
 (segment (start 47.6 58.2) (end 53.1 63.7) (width 0.6) (layer "B.Cu") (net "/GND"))
 (segment (start 40.1 65.099999) (end 40.7 65.099999) (width 0.6) (layer "B.Cu") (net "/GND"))
 (segment (start 24.6 84.7) (end 24.6 84.3) (width 0.6) (layer "B.Cu") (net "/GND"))
 (segment (start 66.099999 72.7) (end 66.099999 84.7) (width 0.6) (layer "F.Cu") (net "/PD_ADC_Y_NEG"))
 (segment (start 65.3 85.2) (end 65.3 87.6) (width 0.6) (layer "F.Cu") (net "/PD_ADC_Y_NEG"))
 (via (at 65.3 85.2) (size 1) (drill 0.4) (layers "F.Cu" "B.Cu") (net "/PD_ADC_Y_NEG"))
 (via (at 65.3 87.6) (size 1) (drill 0.4) (layers "F.Cu" "B.Cu") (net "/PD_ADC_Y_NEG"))
 (segment (start 16.8 87.6) (end 13.3 84.1) (width 0.6) (layer "B.Cu") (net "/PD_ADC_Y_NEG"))
 (segment (start 65.3 87.6) (end 16.8 87.6) (width 0.6) (layer "B.Cu") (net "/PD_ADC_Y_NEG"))
 (segment (start 66.099999 84.7) (end 65.599999 85.2) (width 0.6) (layer "B.Cu") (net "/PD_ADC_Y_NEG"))
 (segment (start 65.599999 85.2) (end 65.3 85.2) (width 0.6) (layer "B.Cu") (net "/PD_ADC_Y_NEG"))
 (segment (start 41.3 51.2) (end 40.9 50.8) (width 0.6) (layer "F.Cu") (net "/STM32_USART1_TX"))
 (segment (start 40.9 50.8) (end 40.9 47) (width 0.6) (layer "F.Cu") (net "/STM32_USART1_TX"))
 (via (at 41.3 51.2) (size 1) (drill 0.4) (layers "F.Cu" "B.Cu") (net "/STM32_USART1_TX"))
 (via (at 40.9 47) (size 1) (drill 0.4) (layers "F.Cu" "B.Cu") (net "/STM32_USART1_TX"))
 (segment (start 40 49.9) (end 41.3 51.2) (width 0.6) (layer "B.Cu") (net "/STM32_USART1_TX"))
 (segment (start 72.6 51.2) (end 72.6 61.9) (width 0.6) (layer "B.Cu") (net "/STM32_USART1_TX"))
 (segment (start 40.9 47) (end 41.3 46.6) (width 0.6) (layer "B.Cu") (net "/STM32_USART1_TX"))
 (segment (start 72.6 61.9) (end 74.3 63.6) (width 0.6) (layer "B.Cu") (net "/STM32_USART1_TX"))
 (segment (start 68 46.6) (end 72.6 51.2) (width 0.6) (layer "B.Cu") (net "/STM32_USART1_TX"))
 (segment (start 41.3 46.6) (end 68 46.6) (width 0.6) (layer "B.Cu") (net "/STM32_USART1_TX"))
 (segment (start 74.3 63.6) (end 74.3 63.8) (width 0.6) (layer "B.Cu") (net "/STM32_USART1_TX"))
 (segment (start 72.6 77.3) (end 74.3 79) (width 0.6) (layer "B.Cu") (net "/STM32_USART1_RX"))
 (segment (start 72.6 69.5) (end 72.6 77.3) (width 0.6) (layer "B.Cu") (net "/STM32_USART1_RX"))
 (segment (start 39 48.4) (end 61 48.4) (width 0.6) (layer "B.Cu") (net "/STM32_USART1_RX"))
 (segment (start 61 48.4) (end 61.9 49.3) (width 0.6) (layer "B.Cu") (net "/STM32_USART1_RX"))
 (segment (start 61.9 49.3) (end 61.9 58.8) (width 0.6) (layer "B.Cu") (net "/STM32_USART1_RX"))
 (segment (start 37.5 49.9) (end 39 48.4) (width 0.6) (layer "B.Cu") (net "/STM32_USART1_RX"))
 (segment (start 61.9 58.8) (end 72.6 69.5) (width 0.6) (layer "B.Cu") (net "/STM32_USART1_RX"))
 (segment (start 23 85.4) (end 24 86.4) (width 0.6) (layer "B.Cu") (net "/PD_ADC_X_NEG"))
 (segment (start 15.9 74) (end 23 81.1) (width 0.6) (layer "B.Cu") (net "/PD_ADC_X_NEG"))
 (segment (start 41.8 72.7) (end 40.1 72.7) (width 0.6) (layer "B.Cu") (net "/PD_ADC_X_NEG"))
 (segment (start 48.7 81.3) (end 65.599999 81.3) (width 0.6) (layer "B.Cu") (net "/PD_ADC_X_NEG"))
 (segment (start 67.6 86.1) (end 67.3 86.4) (width 0.6) (layer "B.Cu") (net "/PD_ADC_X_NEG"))
 (segment (start 40.1 72.7) (end 48.7 81.3) (width 0.6) (layer "B.Cu") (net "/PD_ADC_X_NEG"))
 (segment (start 43.3 74.2) (end 41.8 72.7) (width 0.6) (layer "B.Cu") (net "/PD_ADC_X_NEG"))
 (segment (start 67.3 86.4) (end 43.8 86.4) (width 0.6) (layer "B.Cu") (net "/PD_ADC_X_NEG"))
 (segment (start 67.6 83.3) (end 58.5 74.2) (width 0.6) (layer "B.Cu") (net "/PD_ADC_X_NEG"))
 (segment (start 65.599999 81.3) (end 67.6 83.3) (width 0.6) (layer "B.Cu") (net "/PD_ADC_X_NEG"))
 (segment (start 24 86.4) (end 67.2 86.4) (width 0.6) (layer "B.Cu") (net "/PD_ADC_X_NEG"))
 (segment (start 42.1 84.7) (end 40.1 84.7) (width 0.6) (layer "B.Cu") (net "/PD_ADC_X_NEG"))
 (segment (start 67.2 86.4) (end 67.6 86) (width 0.6) (layer "B.Cu") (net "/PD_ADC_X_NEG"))
 (segment (start 67.6 86) (end 67.6 83.3) (width 0.6) (layer "B.Cu") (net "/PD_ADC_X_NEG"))
 (segment (start 58.5 74.2) (end 43.3 74.2) (width 0.6) (layer "B.Cu") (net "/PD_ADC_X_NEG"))
 (segment (start 23 81.1) (end 23 85.4) (width 0.6) (layer "B.Cu") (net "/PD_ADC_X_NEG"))
 (segment (start 67.6 83.3) (end 67.6 86.1) (width 0.6) (layer "B.Cu") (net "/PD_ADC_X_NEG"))
 (segment (start 43.8 86.4) (end 42.1 84.7) (width 0.6) (layer "B.Cu") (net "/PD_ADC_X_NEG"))
 (segment (start 51.4 86.4) (end 53.1 84.7) (width 0.6) (layer "F.Cu") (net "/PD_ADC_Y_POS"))
 (segment (start 11.6 84.9) (end 13.1 86.4) (width 0.6) (layer "F.Cu") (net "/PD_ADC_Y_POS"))
 (segment (start 53.1 84.7) (end 53.1 72.7) (width 0.6) (layer "F.Cu") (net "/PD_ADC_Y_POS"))
 (segment (start 13.1 86.4) (end 51.4 86.4) (width 0.6) (layer "F.Cu") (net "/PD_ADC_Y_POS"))
 (segment (start 11.6 83.3) (end 11.6 84.9) (width 0.6) (layer "F.Cu") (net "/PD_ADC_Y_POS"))
 (segment (start 13.3 81.6) (end 11.6 83.3) (width 0.6) (layer "F.Cu") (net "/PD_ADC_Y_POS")))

